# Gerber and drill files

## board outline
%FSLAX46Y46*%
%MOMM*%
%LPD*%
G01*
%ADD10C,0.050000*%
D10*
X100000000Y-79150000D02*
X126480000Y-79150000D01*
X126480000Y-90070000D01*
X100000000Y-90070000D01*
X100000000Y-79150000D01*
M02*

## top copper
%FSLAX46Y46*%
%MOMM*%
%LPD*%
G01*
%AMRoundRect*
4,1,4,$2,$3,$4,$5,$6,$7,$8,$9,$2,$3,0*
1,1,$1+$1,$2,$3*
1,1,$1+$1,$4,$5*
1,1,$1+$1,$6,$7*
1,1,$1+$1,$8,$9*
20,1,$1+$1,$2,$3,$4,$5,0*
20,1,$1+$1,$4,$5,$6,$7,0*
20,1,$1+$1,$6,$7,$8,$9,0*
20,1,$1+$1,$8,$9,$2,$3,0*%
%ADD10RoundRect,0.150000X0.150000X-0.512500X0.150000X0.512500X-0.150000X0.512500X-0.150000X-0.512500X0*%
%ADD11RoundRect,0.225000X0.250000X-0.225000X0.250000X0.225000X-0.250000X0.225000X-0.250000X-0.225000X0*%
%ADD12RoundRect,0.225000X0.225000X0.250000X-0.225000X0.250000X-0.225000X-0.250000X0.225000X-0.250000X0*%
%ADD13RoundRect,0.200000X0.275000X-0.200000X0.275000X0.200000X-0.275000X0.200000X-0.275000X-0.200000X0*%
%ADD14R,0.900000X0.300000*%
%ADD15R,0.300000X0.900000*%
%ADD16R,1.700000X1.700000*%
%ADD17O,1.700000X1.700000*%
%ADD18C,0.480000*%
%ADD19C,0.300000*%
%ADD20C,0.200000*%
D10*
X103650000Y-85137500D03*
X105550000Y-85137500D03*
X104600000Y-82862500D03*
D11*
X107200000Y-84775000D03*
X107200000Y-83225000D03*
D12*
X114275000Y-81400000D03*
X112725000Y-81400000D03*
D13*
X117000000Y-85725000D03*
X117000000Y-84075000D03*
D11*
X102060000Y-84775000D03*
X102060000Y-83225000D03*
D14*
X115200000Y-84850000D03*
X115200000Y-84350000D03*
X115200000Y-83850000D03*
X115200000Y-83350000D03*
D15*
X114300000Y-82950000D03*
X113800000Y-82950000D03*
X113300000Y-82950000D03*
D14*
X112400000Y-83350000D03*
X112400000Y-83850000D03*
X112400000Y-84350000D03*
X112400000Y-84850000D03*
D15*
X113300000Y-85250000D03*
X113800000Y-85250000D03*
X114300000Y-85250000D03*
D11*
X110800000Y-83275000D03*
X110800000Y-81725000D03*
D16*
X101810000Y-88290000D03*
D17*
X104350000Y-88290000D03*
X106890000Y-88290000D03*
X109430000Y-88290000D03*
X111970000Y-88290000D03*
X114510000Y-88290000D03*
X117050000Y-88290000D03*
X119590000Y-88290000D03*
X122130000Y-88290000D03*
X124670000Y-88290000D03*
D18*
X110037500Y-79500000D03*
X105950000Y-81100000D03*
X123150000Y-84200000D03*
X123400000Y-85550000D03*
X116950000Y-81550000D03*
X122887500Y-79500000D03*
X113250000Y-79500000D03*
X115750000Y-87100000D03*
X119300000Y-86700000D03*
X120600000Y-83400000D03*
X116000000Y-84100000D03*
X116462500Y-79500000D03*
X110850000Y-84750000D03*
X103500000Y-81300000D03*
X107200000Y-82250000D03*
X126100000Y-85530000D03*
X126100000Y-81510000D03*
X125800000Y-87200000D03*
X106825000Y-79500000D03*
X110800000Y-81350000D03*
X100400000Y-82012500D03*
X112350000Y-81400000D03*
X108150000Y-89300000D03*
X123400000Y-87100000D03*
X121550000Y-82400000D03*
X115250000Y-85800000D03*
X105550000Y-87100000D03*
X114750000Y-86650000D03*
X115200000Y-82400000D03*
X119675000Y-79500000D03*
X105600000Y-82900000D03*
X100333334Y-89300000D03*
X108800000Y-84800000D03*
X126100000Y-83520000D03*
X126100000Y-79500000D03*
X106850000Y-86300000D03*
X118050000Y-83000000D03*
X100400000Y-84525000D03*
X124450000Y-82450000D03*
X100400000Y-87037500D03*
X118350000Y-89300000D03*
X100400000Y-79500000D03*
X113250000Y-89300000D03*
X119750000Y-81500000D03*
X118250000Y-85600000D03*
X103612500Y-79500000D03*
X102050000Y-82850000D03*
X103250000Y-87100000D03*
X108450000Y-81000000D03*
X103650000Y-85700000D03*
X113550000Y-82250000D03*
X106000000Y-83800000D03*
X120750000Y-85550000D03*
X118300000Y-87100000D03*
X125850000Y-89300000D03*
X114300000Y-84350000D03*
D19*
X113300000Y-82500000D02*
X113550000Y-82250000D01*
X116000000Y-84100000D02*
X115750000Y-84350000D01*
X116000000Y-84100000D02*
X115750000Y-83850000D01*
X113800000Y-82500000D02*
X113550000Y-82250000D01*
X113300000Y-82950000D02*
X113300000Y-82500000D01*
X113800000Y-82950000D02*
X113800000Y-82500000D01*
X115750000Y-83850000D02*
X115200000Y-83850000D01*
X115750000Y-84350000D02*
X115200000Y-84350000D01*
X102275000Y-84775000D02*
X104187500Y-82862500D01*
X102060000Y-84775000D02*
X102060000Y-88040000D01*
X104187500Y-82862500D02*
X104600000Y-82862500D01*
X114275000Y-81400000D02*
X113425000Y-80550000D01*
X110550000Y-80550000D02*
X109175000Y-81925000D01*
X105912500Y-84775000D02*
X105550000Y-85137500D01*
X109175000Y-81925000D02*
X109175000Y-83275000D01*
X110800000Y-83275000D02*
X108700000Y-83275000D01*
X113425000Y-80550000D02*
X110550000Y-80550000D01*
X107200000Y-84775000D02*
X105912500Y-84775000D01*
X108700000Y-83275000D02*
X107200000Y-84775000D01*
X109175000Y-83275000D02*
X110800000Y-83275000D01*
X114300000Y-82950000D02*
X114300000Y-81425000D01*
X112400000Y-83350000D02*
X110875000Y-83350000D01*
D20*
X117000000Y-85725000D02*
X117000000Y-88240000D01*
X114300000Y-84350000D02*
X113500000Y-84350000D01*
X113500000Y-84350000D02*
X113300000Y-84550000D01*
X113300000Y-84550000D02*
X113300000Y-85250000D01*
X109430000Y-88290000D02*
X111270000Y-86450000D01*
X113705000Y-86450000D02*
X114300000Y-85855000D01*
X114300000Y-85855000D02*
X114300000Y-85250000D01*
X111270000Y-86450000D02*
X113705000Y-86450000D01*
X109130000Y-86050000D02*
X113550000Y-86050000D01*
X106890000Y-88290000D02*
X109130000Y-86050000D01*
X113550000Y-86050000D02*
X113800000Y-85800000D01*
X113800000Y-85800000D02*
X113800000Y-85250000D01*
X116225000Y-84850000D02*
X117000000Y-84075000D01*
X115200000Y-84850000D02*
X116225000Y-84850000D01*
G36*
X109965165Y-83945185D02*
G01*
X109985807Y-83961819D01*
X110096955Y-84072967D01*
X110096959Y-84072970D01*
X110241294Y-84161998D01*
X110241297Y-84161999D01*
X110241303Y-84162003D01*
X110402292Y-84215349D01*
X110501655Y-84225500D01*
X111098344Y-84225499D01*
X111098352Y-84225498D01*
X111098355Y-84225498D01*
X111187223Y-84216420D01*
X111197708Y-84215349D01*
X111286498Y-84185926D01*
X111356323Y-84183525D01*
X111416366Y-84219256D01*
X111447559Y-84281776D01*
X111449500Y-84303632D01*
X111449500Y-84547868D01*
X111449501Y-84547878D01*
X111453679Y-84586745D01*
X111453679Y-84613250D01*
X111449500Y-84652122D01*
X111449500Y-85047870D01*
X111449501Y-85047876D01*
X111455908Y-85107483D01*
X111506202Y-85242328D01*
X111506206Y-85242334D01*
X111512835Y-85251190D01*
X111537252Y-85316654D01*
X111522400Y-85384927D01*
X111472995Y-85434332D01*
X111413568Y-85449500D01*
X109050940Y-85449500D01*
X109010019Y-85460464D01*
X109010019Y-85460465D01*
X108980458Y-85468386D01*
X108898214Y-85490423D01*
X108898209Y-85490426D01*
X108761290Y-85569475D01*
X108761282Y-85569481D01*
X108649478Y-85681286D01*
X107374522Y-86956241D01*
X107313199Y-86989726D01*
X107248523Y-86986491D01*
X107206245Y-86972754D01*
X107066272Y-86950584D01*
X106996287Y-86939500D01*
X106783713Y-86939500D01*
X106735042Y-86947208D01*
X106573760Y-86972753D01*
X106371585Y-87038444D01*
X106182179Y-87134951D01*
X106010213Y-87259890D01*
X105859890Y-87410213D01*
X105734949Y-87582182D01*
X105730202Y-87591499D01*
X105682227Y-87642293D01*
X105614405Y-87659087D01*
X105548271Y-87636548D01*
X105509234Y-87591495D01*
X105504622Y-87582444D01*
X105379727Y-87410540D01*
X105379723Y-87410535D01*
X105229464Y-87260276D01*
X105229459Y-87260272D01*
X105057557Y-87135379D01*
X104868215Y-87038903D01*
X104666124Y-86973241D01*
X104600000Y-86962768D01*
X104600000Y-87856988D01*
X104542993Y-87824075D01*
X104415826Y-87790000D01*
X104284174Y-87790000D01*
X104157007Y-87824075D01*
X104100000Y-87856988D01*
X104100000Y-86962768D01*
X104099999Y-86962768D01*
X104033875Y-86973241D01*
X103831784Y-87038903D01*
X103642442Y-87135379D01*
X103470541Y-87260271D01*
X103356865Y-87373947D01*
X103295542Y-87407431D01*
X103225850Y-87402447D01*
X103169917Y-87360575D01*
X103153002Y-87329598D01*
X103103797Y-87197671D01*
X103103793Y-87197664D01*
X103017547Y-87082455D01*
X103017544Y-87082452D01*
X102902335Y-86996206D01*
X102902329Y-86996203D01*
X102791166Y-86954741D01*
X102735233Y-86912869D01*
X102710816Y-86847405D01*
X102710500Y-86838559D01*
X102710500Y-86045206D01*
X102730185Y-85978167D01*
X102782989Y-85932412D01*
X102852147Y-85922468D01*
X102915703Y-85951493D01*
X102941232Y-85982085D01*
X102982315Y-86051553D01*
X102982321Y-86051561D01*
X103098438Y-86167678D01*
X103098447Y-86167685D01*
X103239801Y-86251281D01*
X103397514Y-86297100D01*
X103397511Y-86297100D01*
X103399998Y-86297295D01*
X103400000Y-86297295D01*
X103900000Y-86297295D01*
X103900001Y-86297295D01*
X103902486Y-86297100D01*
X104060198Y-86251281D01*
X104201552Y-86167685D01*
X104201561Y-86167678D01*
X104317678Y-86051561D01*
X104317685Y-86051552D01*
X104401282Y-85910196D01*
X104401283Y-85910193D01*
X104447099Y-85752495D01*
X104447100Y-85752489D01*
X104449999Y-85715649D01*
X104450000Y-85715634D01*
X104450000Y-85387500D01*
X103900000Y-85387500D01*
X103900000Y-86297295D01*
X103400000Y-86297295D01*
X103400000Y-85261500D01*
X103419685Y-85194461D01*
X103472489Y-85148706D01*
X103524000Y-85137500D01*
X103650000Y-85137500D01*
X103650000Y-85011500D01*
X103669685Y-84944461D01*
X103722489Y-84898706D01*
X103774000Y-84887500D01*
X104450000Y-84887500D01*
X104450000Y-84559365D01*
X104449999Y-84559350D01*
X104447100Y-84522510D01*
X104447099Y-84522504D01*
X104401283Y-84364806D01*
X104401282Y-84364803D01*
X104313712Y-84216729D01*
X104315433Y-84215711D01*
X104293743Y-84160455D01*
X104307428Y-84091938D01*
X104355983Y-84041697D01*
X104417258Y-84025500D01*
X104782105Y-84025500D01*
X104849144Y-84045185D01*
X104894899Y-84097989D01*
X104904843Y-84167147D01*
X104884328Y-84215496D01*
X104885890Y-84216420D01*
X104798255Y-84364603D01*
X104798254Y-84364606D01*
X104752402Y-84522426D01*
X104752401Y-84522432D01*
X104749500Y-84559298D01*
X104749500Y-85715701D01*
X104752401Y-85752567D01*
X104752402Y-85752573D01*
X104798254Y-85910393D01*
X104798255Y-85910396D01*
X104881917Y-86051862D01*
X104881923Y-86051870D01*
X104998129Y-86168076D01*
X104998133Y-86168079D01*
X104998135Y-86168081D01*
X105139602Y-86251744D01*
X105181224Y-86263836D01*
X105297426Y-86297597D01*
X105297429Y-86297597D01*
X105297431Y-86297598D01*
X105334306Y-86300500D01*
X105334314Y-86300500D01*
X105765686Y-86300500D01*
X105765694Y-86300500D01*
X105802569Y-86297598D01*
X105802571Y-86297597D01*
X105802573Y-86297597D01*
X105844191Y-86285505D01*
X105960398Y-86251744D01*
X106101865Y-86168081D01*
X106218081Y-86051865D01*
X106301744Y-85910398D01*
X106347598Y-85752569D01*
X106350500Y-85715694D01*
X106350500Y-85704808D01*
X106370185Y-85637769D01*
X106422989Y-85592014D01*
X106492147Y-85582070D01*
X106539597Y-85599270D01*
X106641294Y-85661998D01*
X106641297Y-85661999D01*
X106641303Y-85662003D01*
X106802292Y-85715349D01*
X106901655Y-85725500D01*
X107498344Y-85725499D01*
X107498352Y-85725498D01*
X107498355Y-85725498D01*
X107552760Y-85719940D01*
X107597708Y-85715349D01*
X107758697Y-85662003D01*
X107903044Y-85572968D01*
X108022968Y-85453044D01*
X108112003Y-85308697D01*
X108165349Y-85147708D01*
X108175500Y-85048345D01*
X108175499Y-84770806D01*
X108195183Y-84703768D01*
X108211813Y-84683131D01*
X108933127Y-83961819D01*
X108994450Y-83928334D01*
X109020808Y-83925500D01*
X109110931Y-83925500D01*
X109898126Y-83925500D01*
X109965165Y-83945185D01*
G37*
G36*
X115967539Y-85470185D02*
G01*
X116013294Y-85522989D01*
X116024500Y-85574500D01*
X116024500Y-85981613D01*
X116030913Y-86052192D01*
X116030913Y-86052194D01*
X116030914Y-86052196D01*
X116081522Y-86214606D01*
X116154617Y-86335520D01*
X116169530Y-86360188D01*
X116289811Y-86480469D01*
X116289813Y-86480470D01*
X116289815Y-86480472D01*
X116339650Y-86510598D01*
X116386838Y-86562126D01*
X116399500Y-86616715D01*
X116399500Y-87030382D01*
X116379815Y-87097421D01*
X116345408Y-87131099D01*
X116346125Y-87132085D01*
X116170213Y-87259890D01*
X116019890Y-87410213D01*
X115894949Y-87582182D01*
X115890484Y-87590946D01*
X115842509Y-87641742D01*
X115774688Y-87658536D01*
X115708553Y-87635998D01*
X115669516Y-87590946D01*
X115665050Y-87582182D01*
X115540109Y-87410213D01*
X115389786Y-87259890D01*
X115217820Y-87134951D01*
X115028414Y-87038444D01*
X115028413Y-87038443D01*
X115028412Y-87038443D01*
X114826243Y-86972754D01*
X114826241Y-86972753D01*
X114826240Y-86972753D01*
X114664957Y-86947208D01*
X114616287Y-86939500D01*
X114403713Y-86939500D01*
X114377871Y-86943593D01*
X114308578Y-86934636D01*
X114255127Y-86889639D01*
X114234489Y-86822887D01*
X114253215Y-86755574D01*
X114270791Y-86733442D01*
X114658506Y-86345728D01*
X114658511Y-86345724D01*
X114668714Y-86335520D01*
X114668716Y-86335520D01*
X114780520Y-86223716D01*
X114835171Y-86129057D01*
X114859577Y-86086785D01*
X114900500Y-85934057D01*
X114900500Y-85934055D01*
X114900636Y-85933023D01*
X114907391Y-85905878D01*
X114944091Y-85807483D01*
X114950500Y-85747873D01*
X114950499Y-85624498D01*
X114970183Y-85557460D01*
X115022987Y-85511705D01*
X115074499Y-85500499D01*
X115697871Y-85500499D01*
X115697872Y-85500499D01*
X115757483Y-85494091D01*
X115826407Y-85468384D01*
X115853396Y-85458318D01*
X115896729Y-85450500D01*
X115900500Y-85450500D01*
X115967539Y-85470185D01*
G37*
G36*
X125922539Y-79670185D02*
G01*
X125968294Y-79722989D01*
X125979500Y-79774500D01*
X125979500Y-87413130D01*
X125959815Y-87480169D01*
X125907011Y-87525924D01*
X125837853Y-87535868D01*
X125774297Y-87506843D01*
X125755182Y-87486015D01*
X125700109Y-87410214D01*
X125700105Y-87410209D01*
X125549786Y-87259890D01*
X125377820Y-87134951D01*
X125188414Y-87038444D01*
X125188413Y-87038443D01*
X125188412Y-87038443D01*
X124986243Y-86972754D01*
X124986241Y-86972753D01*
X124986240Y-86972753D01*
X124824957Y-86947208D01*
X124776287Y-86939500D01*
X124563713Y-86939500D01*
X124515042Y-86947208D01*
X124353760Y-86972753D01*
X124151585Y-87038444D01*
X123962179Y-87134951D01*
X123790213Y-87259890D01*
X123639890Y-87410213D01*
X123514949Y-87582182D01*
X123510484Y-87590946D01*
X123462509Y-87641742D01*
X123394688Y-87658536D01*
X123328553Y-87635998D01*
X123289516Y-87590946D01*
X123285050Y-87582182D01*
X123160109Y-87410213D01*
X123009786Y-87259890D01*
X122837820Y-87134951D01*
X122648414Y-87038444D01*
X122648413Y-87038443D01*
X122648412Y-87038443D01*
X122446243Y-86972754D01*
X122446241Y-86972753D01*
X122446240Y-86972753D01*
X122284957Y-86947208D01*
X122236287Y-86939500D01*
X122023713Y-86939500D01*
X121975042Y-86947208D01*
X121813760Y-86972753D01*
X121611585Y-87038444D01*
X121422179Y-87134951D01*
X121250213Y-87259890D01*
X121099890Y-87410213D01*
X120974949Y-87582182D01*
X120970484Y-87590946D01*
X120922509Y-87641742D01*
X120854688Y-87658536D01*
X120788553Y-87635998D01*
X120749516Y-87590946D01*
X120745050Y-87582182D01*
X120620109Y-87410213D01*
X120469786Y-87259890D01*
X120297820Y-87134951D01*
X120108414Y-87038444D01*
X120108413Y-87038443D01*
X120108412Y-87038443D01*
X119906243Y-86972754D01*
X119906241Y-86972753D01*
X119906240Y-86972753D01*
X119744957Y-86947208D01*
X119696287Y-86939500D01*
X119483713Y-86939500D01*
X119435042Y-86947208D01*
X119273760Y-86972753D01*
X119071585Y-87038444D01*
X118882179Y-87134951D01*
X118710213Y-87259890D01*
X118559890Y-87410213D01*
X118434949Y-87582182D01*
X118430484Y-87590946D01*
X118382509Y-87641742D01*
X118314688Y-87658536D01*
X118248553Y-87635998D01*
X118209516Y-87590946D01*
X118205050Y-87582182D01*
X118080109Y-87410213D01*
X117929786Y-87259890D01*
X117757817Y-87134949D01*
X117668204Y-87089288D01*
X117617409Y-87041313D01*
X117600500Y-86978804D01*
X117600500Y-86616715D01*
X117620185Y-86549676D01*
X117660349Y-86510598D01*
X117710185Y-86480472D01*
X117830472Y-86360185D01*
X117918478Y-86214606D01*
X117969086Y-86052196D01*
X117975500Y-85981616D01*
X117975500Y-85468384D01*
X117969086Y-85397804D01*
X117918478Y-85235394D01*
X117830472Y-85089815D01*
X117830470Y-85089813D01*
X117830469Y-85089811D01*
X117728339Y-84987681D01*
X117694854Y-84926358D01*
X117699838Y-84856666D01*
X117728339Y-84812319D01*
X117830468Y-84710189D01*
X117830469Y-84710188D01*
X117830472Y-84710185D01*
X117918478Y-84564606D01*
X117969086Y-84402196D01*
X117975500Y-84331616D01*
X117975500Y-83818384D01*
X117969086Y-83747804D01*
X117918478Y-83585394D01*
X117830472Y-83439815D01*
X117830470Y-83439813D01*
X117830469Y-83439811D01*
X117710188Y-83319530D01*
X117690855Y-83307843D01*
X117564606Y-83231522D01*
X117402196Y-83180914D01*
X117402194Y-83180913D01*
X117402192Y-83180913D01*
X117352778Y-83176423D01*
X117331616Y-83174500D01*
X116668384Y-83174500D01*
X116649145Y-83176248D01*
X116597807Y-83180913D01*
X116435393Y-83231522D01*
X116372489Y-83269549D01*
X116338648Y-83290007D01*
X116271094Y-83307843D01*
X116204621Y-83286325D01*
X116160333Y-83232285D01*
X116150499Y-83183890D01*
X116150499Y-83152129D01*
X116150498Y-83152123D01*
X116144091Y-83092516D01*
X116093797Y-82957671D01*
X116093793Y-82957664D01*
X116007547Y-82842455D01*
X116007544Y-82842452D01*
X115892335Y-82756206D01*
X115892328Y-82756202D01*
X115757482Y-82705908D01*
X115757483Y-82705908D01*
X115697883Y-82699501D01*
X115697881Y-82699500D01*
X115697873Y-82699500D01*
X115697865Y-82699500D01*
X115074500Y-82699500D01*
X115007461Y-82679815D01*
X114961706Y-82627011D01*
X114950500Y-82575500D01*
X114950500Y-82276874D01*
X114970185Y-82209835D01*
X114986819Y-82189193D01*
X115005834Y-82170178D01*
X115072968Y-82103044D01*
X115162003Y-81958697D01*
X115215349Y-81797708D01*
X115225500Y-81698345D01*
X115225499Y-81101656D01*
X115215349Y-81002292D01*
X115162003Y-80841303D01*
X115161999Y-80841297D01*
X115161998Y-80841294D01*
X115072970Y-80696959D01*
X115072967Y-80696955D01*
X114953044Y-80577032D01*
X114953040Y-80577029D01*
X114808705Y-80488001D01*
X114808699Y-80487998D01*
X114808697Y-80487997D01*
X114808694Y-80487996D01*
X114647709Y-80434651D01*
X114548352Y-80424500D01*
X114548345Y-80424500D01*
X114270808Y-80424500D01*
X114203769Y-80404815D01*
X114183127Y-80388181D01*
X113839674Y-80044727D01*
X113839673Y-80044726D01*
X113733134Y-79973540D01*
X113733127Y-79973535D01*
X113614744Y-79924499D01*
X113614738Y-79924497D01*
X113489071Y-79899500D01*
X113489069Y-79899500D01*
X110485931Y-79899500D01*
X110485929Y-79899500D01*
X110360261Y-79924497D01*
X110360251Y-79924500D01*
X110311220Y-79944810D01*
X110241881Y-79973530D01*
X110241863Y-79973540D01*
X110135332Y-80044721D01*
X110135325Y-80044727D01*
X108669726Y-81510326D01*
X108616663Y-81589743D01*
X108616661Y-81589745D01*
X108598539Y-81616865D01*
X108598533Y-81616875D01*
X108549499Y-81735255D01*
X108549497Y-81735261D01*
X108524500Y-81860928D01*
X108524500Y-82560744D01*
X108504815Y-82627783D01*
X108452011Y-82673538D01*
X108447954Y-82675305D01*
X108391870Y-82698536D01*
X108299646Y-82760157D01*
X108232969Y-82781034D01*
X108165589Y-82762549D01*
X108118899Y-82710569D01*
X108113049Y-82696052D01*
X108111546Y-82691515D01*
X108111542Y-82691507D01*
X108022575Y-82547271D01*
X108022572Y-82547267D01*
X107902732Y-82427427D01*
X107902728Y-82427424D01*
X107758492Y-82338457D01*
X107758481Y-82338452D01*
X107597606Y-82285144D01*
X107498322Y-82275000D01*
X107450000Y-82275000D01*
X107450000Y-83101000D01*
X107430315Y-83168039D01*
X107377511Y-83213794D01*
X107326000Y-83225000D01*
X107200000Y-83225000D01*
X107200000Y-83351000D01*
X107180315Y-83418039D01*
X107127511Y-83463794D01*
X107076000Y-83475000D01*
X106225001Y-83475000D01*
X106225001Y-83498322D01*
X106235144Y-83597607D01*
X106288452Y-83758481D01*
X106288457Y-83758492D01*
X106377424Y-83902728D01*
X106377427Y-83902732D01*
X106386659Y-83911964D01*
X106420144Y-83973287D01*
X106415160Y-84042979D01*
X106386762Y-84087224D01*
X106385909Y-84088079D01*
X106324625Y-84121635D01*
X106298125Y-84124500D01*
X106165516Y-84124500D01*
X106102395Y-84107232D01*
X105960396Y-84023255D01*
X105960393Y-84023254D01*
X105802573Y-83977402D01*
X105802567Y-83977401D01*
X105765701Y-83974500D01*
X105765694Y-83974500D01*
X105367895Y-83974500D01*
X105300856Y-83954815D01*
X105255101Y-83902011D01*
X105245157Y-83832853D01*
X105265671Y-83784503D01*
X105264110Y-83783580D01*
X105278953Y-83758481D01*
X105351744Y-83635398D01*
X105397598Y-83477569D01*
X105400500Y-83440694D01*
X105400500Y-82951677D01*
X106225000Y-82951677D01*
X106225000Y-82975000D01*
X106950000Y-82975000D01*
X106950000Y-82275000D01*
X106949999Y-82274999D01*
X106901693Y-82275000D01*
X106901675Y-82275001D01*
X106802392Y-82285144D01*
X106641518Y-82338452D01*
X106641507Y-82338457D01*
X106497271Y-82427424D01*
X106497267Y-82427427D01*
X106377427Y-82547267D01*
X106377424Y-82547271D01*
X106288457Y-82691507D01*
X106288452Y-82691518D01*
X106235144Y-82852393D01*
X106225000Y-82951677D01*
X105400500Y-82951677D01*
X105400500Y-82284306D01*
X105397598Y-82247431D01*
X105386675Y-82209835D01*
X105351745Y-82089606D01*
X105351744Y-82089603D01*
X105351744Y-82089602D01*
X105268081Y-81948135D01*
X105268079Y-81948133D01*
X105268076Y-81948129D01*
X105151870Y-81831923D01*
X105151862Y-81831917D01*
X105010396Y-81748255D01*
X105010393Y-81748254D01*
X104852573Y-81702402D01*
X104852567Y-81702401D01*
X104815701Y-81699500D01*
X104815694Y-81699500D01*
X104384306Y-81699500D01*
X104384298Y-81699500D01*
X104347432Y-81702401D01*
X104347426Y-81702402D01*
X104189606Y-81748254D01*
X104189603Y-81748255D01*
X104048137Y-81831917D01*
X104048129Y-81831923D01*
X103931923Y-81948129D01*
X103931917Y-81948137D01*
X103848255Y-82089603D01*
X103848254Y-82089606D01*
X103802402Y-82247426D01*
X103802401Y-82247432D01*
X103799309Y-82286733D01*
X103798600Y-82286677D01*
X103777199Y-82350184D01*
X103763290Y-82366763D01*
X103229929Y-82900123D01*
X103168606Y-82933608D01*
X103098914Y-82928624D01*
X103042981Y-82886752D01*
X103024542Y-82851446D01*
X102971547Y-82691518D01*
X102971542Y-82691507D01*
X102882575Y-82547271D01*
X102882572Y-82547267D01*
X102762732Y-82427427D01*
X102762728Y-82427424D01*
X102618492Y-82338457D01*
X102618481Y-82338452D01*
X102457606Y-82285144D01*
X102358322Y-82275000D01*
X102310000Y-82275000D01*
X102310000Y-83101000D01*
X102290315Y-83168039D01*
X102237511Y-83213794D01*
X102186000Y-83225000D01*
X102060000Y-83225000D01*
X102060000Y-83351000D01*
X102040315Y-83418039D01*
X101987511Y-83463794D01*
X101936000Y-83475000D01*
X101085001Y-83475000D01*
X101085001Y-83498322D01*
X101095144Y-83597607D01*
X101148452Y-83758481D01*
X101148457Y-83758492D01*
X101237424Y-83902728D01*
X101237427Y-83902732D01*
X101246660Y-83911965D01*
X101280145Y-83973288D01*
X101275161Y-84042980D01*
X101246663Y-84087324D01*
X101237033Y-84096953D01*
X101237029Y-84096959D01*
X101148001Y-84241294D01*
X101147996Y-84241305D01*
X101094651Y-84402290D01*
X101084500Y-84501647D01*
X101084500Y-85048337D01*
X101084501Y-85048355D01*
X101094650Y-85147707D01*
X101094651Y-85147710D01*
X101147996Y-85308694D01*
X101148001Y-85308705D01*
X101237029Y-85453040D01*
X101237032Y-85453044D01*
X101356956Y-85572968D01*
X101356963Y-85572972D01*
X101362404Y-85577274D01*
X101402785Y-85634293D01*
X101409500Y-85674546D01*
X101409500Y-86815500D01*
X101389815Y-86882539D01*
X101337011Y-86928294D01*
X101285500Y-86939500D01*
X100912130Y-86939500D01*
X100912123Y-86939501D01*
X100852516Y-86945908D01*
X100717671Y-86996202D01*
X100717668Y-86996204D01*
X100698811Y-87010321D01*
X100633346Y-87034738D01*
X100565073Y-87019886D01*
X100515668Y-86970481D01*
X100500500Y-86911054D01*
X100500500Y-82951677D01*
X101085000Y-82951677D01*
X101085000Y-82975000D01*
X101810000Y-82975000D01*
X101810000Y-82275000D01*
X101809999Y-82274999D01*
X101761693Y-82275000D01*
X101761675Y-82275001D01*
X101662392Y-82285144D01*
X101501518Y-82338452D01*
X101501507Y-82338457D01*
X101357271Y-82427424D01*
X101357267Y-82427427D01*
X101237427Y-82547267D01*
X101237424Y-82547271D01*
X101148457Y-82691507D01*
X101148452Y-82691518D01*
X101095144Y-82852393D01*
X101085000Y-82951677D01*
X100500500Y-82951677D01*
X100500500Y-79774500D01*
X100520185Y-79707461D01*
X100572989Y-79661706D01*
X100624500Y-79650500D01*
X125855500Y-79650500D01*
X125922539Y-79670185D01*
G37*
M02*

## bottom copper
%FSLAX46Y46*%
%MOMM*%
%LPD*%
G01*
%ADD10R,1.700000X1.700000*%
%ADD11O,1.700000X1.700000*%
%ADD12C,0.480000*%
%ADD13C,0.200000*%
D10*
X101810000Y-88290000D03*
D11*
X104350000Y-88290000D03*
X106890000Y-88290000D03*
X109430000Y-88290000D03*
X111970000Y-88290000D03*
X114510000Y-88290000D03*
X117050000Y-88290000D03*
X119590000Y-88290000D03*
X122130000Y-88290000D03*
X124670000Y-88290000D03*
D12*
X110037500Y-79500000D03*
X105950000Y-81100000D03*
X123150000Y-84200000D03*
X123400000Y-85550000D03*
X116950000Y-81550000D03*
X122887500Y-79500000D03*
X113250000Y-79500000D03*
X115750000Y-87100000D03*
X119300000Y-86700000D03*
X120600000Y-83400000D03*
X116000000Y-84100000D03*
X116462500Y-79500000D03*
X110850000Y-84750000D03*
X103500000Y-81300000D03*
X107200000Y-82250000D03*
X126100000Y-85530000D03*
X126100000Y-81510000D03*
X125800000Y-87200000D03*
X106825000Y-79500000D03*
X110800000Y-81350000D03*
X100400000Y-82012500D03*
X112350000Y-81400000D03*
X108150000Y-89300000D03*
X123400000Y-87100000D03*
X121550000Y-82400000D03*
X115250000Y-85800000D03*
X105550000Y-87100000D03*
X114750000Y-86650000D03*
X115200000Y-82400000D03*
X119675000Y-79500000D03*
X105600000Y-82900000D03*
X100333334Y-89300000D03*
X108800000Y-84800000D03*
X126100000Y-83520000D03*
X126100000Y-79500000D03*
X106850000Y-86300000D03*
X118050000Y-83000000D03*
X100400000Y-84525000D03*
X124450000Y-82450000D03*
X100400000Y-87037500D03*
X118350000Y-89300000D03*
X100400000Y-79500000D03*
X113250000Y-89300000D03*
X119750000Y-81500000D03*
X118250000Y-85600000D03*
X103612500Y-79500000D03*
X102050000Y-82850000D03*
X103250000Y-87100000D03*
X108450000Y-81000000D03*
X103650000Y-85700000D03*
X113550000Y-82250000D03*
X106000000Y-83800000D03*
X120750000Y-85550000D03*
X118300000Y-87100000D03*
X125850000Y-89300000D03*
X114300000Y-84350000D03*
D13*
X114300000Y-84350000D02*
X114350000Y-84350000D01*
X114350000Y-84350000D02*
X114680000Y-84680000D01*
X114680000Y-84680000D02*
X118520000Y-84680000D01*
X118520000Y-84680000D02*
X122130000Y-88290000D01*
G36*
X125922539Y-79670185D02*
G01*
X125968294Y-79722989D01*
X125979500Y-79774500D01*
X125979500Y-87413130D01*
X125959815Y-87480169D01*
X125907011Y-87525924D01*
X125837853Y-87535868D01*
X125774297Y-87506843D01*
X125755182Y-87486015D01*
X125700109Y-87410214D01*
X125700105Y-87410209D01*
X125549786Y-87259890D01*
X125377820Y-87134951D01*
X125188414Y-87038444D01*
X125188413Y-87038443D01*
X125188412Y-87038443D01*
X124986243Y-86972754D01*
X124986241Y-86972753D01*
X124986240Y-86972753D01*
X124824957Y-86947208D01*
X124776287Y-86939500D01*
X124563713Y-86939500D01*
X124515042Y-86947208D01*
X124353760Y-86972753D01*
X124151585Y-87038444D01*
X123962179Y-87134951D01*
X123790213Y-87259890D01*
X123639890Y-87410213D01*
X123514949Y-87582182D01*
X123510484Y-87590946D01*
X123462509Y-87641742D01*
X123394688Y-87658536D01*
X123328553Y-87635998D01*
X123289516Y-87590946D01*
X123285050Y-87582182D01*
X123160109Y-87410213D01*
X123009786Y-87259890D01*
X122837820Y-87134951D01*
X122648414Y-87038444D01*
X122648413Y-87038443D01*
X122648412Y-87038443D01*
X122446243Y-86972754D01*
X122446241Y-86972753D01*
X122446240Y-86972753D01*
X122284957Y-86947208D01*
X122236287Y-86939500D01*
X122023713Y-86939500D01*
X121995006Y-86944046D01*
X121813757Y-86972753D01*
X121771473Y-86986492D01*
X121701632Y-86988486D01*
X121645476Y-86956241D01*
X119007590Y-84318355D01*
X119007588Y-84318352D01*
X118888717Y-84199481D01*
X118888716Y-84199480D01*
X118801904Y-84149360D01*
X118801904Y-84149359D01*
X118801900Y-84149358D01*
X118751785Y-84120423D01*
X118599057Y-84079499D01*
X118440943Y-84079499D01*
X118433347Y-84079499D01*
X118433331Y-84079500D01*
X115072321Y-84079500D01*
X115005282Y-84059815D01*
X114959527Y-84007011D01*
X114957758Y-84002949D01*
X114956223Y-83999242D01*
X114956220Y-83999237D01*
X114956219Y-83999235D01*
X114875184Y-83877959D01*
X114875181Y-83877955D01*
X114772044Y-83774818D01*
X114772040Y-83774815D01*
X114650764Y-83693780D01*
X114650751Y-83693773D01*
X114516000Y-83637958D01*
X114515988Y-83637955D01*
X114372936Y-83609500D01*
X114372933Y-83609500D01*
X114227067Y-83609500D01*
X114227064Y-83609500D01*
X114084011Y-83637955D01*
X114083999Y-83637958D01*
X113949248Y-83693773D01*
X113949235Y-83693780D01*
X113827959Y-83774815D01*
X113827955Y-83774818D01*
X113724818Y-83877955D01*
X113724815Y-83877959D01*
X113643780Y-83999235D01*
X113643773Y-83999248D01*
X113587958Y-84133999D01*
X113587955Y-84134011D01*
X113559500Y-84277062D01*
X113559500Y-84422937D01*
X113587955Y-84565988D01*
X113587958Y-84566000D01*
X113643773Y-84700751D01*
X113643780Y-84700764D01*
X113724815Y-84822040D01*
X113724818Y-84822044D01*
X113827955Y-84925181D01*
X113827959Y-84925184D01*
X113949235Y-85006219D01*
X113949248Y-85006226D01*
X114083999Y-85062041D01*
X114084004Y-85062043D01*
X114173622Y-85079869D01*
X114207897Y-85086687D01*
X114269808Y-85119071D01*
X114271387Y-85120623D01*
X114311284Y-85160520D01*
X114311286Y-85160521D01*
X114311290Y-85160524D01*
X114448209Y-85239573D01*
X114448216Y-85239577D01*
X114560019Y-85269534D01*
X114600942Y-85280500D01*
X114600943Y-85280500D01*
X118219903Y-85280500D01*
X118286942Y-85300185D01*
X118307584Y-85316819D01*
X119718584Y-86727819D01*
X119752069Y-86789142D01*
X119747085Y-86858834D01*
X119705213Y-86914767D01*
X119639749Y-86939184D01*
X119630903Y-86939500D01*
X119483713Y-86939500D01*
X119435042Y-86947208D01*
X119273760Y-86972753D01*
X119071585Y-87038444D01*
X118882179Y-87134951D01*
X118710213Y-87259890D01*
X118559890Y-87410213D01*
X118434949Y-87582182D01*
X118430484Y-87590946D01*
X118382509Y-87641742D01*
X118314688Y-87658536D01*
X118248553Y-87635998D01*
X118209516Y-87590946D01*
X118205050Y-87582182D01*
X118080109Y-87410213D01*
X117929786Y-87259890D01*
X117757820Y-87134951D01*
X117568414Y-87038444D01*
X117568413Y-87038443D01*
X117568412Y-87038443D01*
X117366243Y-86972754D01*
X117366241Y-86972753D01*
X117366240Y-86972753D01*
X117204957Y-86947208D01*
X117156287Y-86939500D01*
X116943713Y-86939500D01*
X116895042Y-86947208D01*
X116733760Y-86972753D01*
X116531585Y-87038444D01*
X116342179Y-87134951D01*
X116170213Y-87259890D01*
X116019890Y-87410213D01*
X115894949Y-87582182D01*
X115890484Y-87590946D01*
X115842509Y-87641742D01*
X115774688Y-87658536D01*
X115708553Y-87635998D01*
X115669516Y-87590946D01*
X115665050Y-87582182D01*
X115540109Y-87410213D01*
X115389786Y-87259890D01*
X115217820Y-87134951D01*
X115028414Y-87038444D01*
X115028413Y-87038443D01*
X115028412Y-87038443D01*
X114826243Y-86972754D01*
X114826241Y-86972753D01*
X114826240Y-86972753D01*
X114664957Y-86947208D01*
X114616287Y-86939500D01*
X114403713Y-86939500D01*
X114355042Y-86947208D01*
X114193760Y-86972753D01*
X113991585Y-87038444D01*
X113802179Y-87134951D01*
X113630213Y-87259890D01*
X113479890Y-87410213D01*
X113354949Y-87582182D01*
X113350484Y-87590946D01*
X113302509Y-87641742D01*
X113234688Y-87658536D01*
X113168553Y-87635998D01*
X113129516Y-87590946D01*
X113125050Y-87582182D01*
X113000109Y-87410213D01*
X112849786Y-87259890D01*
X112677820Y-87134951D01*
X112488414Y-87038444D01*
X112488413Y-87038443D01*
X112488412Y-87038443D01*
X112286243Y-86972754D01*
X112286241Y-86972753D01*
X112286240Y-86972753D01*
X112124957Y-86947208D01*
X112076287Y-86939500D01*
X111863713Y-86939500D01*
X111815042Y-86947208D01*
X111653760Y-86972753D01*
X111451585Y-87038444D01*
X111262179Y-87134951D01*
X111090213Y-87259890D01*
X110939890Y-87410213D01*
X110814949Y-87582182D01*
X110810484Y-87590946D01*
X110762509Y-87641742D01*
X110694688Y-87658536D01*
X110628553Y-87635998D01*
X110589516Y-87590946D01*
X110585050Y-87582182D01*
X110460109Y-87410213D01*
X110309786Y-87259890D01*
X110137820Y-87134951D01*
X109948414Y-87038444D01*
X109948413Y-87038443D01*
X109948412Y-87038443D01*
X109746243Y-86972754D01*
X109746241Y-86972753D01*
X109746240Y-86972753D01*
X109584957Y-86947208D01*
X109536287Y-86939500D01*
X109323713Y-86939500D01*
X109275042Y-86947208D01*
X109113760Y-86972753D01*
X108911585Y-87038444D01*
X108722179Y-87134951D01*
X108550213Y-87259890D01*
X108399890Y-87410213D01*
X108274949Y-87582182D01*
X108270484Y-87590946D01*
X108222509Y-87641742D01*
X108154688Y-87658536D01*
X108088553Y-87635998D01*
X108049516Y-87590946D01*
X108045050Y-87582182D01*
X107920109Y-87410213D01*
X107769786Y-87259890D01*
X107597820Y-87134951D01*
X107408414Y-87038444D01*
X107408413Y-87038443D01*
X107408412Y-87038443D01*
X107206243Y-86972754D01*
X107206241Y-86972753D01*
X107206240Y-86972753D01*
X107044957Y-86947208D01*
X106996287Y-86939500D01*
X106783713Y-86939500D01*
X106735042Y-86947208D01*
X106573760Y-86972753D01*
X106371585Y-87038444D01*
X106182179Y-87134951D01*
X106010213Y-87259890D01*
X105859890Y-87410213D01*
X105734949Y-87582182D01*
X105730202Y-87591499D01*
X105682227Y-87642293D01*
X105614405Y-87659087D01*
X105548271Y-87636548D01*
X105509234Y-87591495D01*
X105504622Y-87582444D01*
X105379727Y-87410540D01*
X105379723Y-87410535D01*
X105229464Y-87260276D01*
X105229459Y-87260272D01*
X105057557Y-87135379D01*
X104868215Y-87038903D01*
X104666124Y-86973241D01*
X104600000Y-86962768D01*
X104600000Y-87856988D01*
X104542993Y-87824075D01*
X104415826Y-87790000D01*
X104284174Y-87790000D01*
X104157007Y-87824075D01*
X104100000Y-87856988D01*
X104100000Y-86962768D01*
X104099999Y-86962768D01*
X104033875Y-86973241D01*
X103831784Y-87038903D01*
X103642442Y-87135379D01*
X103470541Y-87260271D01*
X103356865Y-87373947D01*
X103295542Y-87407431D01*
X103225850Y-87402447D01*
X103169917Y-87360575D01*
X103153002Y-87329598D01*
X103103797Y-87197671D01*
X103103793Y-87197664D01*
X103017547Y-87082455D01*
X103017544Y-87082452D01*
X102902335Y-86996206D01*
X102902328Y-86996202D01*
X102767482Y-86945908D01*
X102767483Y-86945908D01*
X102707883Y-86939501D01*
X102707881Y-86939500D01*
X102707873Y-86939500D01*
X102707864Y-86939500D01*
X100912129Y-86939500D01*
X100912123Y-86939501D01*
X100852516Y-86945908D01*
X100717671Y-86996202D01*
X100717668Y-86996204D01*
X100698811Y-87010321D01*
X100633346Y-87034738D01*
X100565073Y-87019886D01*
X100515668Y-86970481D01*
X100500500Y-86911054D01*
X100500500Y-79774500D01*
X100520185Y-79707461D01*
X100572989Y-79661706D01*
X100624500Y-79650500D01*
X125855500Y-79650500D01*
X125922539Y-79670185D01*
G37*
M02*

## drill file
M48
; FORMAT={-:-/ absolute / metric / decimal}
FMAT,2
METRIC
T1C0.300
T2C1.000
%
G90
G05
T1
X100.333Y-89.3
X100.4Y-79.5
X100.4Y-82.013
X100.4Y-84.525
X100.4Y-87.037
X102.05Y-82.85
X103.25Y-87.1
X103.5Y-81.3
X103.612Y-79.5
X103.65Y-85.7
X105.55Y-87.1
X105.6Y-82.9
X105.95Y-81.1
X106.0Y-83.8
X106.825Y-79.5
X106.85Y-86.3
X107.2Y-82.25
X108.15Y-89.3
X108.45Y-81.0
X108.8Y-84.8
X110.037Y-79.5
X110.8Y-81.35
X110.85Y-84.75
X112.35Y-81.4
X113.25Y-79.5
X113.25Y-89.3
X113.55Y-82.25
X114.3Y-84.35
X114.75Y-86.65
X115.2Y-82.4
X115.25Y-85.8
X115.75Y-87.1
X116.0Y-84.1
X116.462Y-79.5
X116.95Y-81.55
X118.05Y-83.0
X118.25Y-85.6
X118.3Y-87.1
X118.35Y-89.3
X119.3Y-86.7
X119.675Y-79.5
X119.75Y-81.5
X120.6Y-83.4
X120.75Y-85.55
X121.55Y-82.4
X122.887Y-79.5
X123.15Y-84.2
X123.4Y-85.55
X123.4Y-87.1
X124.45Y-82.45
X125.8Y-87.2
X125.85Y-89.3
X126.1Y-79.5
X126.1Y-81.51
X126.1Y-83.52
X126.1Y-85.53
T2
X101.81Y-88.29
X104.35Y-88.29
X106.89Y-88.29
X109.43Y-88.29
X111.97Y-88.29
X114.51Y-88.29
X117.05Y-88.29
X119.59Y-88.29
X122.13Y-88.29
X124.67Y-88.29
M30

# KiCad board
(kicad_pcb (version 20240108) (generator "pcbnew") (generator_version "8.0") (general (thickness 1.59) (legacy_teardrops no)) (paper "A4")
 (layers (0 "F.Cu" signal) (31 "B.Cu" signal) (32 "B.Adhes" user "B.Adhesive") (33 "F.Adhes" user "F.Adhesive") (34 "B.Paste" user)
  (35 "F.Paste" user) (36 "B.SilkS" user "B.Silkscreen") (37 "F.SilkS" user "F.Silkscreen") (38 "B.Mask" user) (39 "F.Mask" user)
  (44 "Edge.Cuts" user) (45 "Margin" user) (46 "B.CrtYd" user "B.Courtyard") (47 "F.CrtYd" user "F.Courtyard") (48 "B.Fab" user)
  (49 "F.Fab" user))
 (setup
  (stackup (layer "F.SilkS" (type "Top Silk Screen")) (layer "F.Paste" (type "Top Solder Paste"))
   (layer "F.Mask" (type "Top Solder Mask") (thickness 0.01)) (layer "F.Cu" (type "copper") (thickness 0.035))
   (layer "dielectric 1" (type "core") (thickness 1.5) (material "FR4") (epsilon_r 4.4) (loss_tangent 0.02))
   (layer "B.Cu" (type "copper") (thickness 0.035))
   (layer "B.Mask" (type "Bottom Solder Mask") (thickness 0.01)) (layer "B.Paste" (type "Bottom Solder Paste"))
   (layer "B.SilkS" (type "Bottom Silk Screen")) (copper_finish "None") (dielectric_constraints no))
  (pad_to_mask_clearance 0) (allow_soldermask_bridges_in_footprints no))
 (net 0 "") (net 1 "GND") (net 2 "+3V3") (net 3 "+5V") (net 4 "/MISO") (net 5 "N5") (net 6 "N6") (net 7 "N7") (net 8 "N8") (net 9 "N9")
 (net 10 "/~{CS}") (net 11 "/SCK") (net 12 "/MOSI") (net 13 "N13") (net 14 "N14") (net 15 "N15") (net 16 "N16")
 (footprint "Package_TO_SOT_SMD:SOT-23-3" (layer "F.Cu") (at 104.6 84 90)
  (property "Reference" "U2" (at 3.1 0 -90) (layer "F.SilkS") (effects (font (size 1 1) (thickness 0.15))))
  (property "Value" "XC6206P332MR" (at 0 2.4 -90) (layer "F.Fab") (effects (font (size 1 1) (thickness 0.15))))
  (pad "1" smd roundrect (at -1.1375 -0.95 90) (size 1.325 0.6) (layers "F.Cu" "F.Paste" "F.Mask") (roundrect_rratio 0.25) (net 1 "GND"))
  (pad "2" smd roundrect (at -1.1375 0.95 90) (size 1.325 0.6) (layers "F.Cu" "F.Paste" "F.Mask") (roundrect_rratio 0.25) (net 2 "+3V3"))
  (pad "3" smd roundrect (at 1.1375 0 90) (size 1.325 0.6) (layers "F.Cu" "F.Paste" "F.Mask") (roundrect_rratio 0.25) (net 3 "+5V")))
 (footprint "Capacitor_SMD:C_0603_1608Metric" (layer "F.Cu") (at 107.2 84 90)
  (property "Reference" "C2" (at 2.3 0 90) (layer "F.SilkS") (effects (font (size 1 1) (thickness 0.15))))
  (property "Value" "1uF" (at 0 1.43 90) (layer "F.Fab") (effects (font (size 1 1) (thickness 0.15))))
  (pad "1" smd roundrect (at -0.775 0 90) (size 0.9 0.95) (layers "F.Cu" "F.Paste" "F.Mask") (roundrect_rratio 0.25) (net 2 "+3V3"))
  (pad "2" smd roundrect (at 0.775 0 90) (size 0.9 0.95) (layers "F.Cu" "F.Paste" "F.Mask") (roundrect_rratio 0.25) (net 1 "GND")))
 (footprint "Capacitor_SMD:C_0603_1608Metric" (layer "F.Cu") (at 113.5 81.4 180)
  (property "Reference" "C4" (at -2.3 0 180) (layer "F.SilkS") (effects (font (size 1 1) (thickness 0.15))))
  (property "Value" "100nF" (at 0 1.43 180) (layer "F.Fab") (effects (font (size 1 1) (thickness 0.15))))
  (pad "1" smd roundrect (at -0.775 0 180) (size 0.9 0.95) (layers "F.Cu" "F.Paste" "F.Mask") (roundrect_rratio 0.25) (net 2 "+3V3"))
  (pad "2" smd roundrect (at 0.775 0 180) (size 0.9 0.95) (layers "F.Cu" "F.Paste" "F.Mask") (roundrect_rratio 0.25) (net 1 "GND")))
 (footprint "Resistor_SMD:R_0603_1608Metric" (layer "F.Cu") (at 117 84.9 90)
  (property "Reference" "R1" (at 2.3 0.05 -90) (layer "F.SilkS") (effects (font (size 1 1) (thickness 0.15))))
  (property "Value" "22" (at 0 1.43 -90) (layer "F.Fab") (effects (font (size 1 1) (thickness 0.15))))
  (pad "1" smd roundrect (at -0.825 0 90) (size 0.8 0.95) (layers "F.Cu" "F.Paste" "F.Mask") (roundrect_rratio 0.25) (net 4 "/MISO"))
  (pad "2" smd roundrect (at 0.825 0 90) (size 0.8 0.95) (layers "F.Cu" "F.Paste" "F.Mask") (roundrect_rratio 0.25) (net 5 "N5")))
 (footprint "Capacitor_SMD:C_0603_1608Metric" (layer "F.Cu") (at 102.06 84 90)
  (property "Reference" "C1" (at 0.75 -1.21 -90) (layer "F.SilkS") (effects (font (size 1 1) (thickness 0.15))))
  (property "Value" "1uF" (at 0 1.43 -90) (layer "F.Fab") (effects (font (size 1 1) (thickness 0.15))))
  (pad "1" smd roundrect (at -0.775 0 90) (size 0.9 0.95) (layers "F.Cu" "F.Paste" "F.Mask") (roundrect_rratio 0.25) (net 3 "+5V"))
  (pad "2" smd roundrect (at 0.775 0 90) (size 0.9 0.95) (layers "F.Cu" "F.Paste" "F.Mask") (roundrect_rratio 0.25) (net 1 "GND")))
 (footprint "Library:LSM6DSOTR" (layer "F.Cu") (at 113.8 84.1 180)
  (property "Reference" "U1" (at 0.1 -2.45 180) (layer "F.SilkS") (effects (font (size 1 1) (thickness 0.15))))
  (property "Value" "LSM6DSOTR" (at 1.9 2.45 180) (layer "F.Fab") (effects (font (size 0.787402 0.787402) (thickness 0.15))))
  (pad "1" smd rect (at -1.4 -0.75 180) (size 0.9 0.3) (layers "F.Cu") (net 5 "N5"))
  (pad "2" smd rect (at -1.4 -0.25 180) (size 0.9 0.3) (layers "F.Cu") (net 1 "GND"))
  (pad "3" smd rect (at -1.4 0.25 180) (size 0.9 0.3) (layers "F.Cu") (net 1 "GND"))
  (pad "4" smd rect (at -1.4 0.75 180) (size 0.9 0.3) (layers "F.Cu") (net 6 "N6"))
  (pad "5" smd rect (at -0.5 1.15 180) (size 0.3 0.9) (layers "F.Cu") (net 2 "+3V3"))
  (pad "6" smd rect (at 0 1.15 180) (size 0.3 0.9) (layers "F.Cu") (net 1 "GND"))
  (pad "7" smd rect (at 0.5 1.15 180) (size 0.3 0.9) (layers "F.Cu") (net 1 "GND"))
  (pad "8" smd rect (at 1.4 0.75 180) (size 0.9 0.3) (layers "F.Cu") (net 2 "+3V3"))
  (pad "9" smd rect (at 1.4 0.25 180) (size 0.9 0.3) (layers "F.Cu") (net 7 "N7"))
  (pad "10" smd rect (at 1.4 -0.25 180) (size 0.9 0.3) (layers "F.Cu") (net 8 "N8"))
  (pad "11" smd rect (at 1.4 -0.75 180) (size 0.9 0.3) (layers "F.Cu") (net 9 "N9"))
  (pad "12" smd rect (at 0.5 -1.15 180) (size 0.3 0.9) (layers "F.Cu") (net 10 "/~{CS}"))
  (pad "13" smd rect (at 0 -1.15 180) (size 0.3 0.9) (layers "F.Cu") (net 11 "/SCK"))
  (pad "14" smd rect (at -0.5 -1.15 180) (size 0.3 0.9) (layers "F.Cu") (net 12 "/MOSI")))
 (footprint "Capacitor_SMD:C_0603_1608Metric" (layer "F.Cu") (at 110.8 82.5 90)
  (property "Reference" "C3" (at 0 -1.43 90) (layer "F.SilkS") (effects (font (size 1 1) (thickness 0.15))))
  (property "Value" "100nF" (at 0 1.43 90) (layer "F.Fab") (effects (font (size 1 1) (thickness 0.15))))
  (pad "1" smd roundrect (at -0.775 0 90) (size 0.9 0.95) (layers "F.Cu" "F.Paste" "F.Mask") (roundrect_rratio 0.25) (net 2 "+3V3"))
  (pad "2" smd roundrect (at 0.775 0 90) (size 0.9 0.95) (layers "F.Cu" "F.Paste" "F.Mask") (roundrect_rratio 0.25) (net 1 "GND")))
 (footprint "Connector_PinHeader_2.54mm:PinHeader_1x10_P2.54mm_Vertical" (layer "B.Cu") (at 101.81 88.29 -90)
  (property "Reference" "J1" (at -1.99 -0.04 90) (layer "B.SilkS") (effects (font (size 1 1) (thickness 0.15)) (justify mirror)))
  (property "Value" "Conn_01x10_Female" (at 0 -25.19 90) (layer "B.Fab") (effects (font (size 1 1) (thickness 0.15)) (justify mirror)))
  (pad "1" thru_hole rect (at 0 0 270) (size 1.7 1.7) (drill 1) (layers "*.Cu" "*.Mask") (remove_unused_layers no) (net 3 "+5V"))
  (pad "2" thru_hole oval (at 0 -2.54 270) (size 1.7 1.7) (drill 1) (layers "*.Cu" "*.Mask") (remove_unused_layers no) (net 1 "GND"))
  (pad "3" thru_hole oval (at 0 -5.08 270) (size 1.7 1.7) (drill 1) (layers "*.Cu" "*.Mask") (remove_unused_layers no) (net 11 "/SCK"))
  (pad "4" thru_hole oval (at 0 -7.62 270) (size 1.7 1.7) (drill 1) (layers "*.Cu" "*.Mask") (remove_unused_layers no) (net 12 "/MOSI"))
  (pad "5" thru_hole oval (at 0 -10.16 270) (size 1.7 1.7) (drill 1) (layers "*.Cu" "*.Mask") (remove_unused_layers no) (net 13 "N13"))
  (pad "6" thru_hole oval (at 0 -12.7 270) (size 1.7 1.7) (drill 1) (layers "*.Cu" "*.Mask") (remove_unused_layers no) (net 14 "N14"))
  (pad "7" thru_hole oval (at 0 -15.24 270) (size 1.7 1.7) (drill 1) (layers "*.Cu" "*.Mask") (remove_unused_layers no) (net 4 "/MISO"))
  (pad "8" thru_hole oval (at 0 -17.78 270) (size 1.7 1.7) (drill 1) (layers "*.Cu" "*.Mask") (remove_unused_layers no) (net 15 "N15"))
  (pad "9" thru_hole oval (at 0 -20.32 270) (size 1.7 1.7) (drill 1) (layers "*.Cu" "*.Mask") (remove_unused_layers no) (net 10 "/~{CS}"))
  (pad "10" thru_hole oval (at 0 -22.86 270) (size 1.7 1.7) (drill 1) (layers "*.Cu" "*.Mask") (remove_unused_layers no) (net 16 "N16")))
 (gr_rect (start 100 79.15) (end 126.48 90.07) (stroke (width 0.05) (type default)) (fill none) (layer "Edge.Cuts"))
 (segment (start 113.3 82.5) (end 113.55 82.25) (width 0.3) (layer "F.Cu") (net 1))
 (segment (start 116 84.1) (end 115.75 84.35) (width 0.3) (layer "F.Cu") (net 1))
 (segment (start 116 84.1) (end 115.75 83.85) (width 0.3) (layer "F.Cu") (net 1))
 (segment (start 113.8 82.5) (end 113.55 82.25) (width 0.3) (layer "F.Cu") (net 1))
 (segment (start 113.3 82.95) (end 113.3 82.5) (width 0.3) (layer "F.Cu") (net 1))
 (segment (start 113.8 82.95) (end 113.8 82.5) (width 0.3) (layer "F.Cu") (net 1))
 (segment (start 115.75 83.85) (end 115.2 83.85) (width 0.3) (layer "F.Cu") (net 1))
 (segment (start 115.75 84.35) (end 115.2 84.35) (width 0.3) (layer "F.Cu") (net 1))
 (via (at 110.0375 79.5) (size 0.48) (drill 0.3) (layers "F.Cu" "B.Cu") (free yes) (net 1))
 (via (at 105.95 81.1) (size 0.48) (drill 0.3) (layers "F.Cu" "B.Cu") (free yes) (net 1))
 (via (at 123.15 84.2) (size 0.48) (drill 0.3) (layers "F.Cu" "B.Cu") (free yes) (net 1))
 (via (at 123.4 85.55) (size 0.48) (drill 0.3) (layers "F.Cu" "B.Cu") (free yes) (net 1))
 (via (at 116.95 81.55) (size 0.48) (drill 0.3) (layers "F.Cu" "B.Cu") (free yes) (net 1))
 (via (at 122.8875 79.5) (size 0.48) (drill 0.3) (layers "F.Cu" "B.Cu") (free yes) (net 1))
 (via (at 113.25 79.5) (size 0.48) (drill 0.3) (layers "F.Cu" "B.Cu") (free yes) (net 1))
 (via (at 115.75 87.1) (size 0.48) (drill 0.3) (layers "F.Cu" "B.Cu") (free yes) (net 1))
 (via (at 119.3 86.7) (size 0.48) (drill 0.3) (layers "F.Cu" "B.Cu") (free yes) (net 1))
 (via (at 120.6 83.4) (size 0.48) (drill 0.3) (layers "F.Cu" "B.Cu") (free yes) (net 1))
 (via (at 116 84.1) (size 0.48) (drill 0.3) (layers "F.Cu" "B.Cu") (free yes) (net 1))
 (via (at 116.4625 79.5) (size 0.48) (drill 0.3) (layers "F.Cu" "B.Cu") (free yes) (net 1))
 (via (at 110.85 84.75) (size 0.48) (drill 0.3) (layers "F.Cu" "B.Cu") (free yes) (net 1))
 (via (at 103.5 81.3) (size 0.48) (drill 0.3) (layers "F.Cu" "B.Cu") (free yes) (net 1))
 (via (at 107.2 82.25) (size 0.48) (drill 0.3) (layers "F.Cu" "B.Cu") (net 1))
 (via (at 126.1 85.53) (size 0.48) (drill 0.3) (layers "F.Cu" "B.Cu") (free yes) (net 1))
 (via (at 126.1 81.51) (size 0.48) (drill 0.3) (layers "F.Cu" "B.Cu") (free yes) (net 1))
 (via (at 125.8 87.2) (size 0.48) (drill 0.3) (layers "F.Cu" "B.Cu") (free yes) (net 1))
 (via (at 106.825 79.5) (size 0.48) (drill 0.3) (layers "F.Cu" "B.Cu") (free yes) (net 1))
 (via (at 110.8 81.35) (size 0.48) (drill 0.3) (layers "F.Cu" "B.Cu") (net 1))
 (via (at 100.4 82.0125) (size 0.48) (drill 0.3) (layers "F.Cu" "B.Cu") (free yes) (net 1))
 (via (at 112.35 81.4) (size 0.48) (drill 0.3) (layers "F.Cu" "B.Cu") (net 1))
 (via (at 108.15 89.3) (size 0.48) (drill 0.3) (layers "F.Cu" "B.Cu") (free yes) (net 1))
 (via (at 123.4 87.1) (size 0.48) (drill 0.3) (layers "F.Cu" "B.Cu") (free yes) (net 1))
 (via (at 121.55 82.4) (size 0.48) (drill 0.3) (layers "F.Cu" "B.Cu") (free yes) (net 1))
 (via (at 115.25 85.8) (size 0.48) (drill 0.3) (layers "F.Cu" "B.Cu") (free yes) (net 1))
 (via (at 105.55 87.1) (size 0.48) (drill 0.3) (layers "F.Cu" "B.Cu") (free yes) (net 1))
 (via (at 114.75 86.65) (size 0.48) (drill 0.3) (layers "F.Cu" "B.Cu") (free yes) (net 1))
 (via (at 115.2 82.4) (size 0.48) (drill 0.3) (layers "F.Cu" "B.Cu") (free yes) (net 1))
 (via (at 119.675 79.5) (size 0.48) (drill 0.3) (layers "F.Cu" "B.Cu") (free yes) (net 1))
 (via (at 105.6 82.9) (size 0.48) (drill 0.3) (layers "F.Cu" "B.Cu") (free yes) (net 1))
 (via (at 100.333334 89.3) (size 0.48) (drill 0.3) (layers "F.Cu" "B.Cu") (free yes) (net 1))
 (via (at 108.8 84.8) (size 0.48) (drill 0.3) (layers "F.Cu" "B.Cu") (free yes) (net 1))
 (via (at 126.1 83.52) (size 0.48) (drill 0.3) (layers "F.Cu" "B.Cu") (free yes) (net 1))
 (via (at 126.1 79.5) (size 0.48) (drill 0.3) (layers "F.Cu" "B.Cu") (free yes) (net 1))
 (via (at 106.85 86.3) (size 0.48) (drill 0.3) (layers "F.Cu" "B.Cu") (free yes) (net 1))
 (via (at 118.05 83) (size 0.48) (drill 0.3) (layers "F.Cu" "B.Cu") (free yes) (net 1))
 (via (at 100.4 84.525) (size 0.48) (drill 0.3) (layers "F.Cu" "B.Cu") (free yes) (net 1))
 (via (at 124.45 82.45) (size 0.48) (drill 0.3) (layers "F.Cu" "B.Cu") (free yes) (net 1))
 (via (at 100.4 87.0375) (size 0.48) (drill 0.3) (layers "F.Cu" "B.Cu") (free yes) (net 1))
 (via (at 118.35 89.3) (size 0.48) (drill 0.3) (layers "F.Cu" "B.Cu") (free yes) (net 1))
 (via (at 100.4 79.5) (size 0.48) (drill 0.3) (layers "F.Cu" "B.Cu") (free yes) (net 1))
 (via (at 113.25 89.3) (size 0.48) (drill 0.3) (layers "F.Cu" "B.Cu") (free yes) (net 1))
 (via (at 119.75 81.5) (size 0.48) (drill 0.3) (layers "F.Cu" "B.Cu") (free yes) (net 1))
 (via (at 118.25 85.6) (size 0.48) (drill 0.3) (layers "F.Cu" "B.Cu") (free yes) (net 1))
 (via (at 103.6125 79.5) (size 0.48) (drill 0.3) (layers "F.Cu" "B.Cu") (free yes) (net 1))
 (via (at 102.05 82.85) (size 0.48) (drill 0.3) (layers "F.Cu" "B.Cu") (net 1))
 (via (at 103.25 87.1) (size 0.48) (drill 0.3) (layers "F.Cu" "B.Cu") (free yes) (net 1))
 (via (at 108.45 81) (size 0.48) (drill 0.3) (layers "F.Cu" "B.Cu") (free yes) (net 1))
 (via (at 103.65 85.7) (size 0.48) (drill 0.3) (layers "F.Cu" "B.Cu") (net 1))
 (via (at 113.55 82.25) (size 0.48) (drill 0.3) (layers "F.Cu" "B.Cu") (free yes) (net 1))
 (via (at 106 83.8) (size 0.48) (drill 0.3) (layers "F.Cu" "B.Cu") (free yes) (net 1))
 (via (at 120.75 85.55) (size 0.48) (drill 0.3) (layers "F.Cu" "B.Cu") (free yes) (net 1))
 (via (at 118.3 87.1) (size 0.48) (drill 0.3) (layers "F.Cu" "B.Cu") (free yes) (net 1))
 (via (at 125.85 89.3) (size 0.48) (drill 0.3) (layers "F.Cu" "B.Cu") (free yes) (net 1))
 (segment (start 102.275 84.775) (end 104.1875 82.8625) (width 0.3) (layer "F.Cu") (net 3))
 (segment (start 102.06 84.775) (end 102.06 88.04) (width 0.3) (layer "F.Cu") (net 3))
 (segment (start 104.1875 82.8625) (end 104.6 82.8625) (width 0.3) (layer "F.Cu") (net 3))
 (segment (start 114.275 81.4) (end 113.425 80.55) (width 0.3) (layer "F.Cu") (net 2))
 (segment (start 110.55 80.55) (end 109.175 81.925) (width 0.3) (layer "F.Cu") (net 2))
 (segment (start 105.9125 84.775) (end 105.55 85.1375) (width 0.3) (layer "F.Cu") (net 2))
 (segment (start 109.175 81.925) (end 109.175 83.275) (width 0.3) (layer "F.Cu") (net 2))
 (segment (start 110.8 83.275) (end 108.7 83.275) (width 0.3) (layer "F.Cu") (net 2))
 (segment (start 113.425 80.55) (end 110.55 80.55) (width 0.3) (layer "F.Cu") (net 2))
 (segment (start 107.2 84.775) (end 105.9125 84.775) (width 0.3) (layer "F.Cu") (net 2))
 (segment (start 108.7 83.275) (end 107.2 84.775) (width 0.3) (layer "F.Cu") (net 2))
 (segment (start 109.175 83.275) (end 110.8 83.275) (width 0.3) (layer "F.Cu") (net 2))
 (segment (start 114.3 82.95) (end 114.3 81.425) (width 0.3) (layer "F.Cu") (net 2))
 (segment (start 112.4 83.35) (end 110.875 83.35) (width 0.3) (layer "F.Cu") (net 2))
 (segment (start 117 85.725) (end 117 88.24) (width 0.2) (layer "F.Cu") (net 4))
 (segment (start 114.3 84.35) (end 113.5 84.35) (width 0.2) (layer "F.Cu") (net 10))
 (segment (start 113.5 84.35) (end 113.3 84.55) (width 0.2) (layer "F.Cu") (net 10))
 (segment (start 113.3 84.55) (end 113.3 85.25) (width 0.2) (layer "F.Cu") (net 10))
 (via (at 114.3 84.35) (size 0.48) (drill 0.3) (layers "F.Cu" "B.Cu") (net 10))
 (segment (start 114.3 84.35) (end 114.35 84.35) (width 0.2) (layer "B.Cu") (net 10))
 (segment (start 114.35 84.35) (end 114.68 84.68) (width 0.2) (layer "B.Cu") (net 10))
 (segment (start 114.68 84.68) (end 118.52 84.68) (width 0.2) (layer "B.Cu") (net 10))
 (segment (start 118.52 84.68) (end 122.13 88.29) (width 0.2) (layer "B.Cu") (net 10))
 (segment (start 109.43 88.29) (end 111.27 86.45) (width 0.2) (layer "F.Cu") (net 12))
 (segment (start 113.705 86.45) (end 114.3 85.855) (width 0.2) (layer "F.Cu") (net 12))
 (segment (start 114.3 85.855) (end 114.3 85.25) (width 0.2) (layer "F.Cu") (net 12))
 (segment (start 111.27 86.45) (end 113.705 86.45) (width 0.2) (layer "F.Cu") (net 12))
 (segment (start 109.13 86.05) (end 113.55 86.05) (width 0.2) (layer "F.Cu") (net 11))
 (segment (start 106.89 88.29) (end 109.13 86.05) (width 0.2) (layer "F.Cu") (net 11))
 (segment (start 113.55 86.05) (end 113.8 85.8) (width 0.2) (layer "F.Cu") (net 11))
 (segment (start 113.8 85.8) (end 113.8 85.25) (width 0.2) (layer "F.Cu") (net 11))
 (segment (start 116.225 84.85) (end 117 84.075) (width 0.2) (layer "F.Cu") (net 5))
 (segment (start 115.2 84.85) (end 116.225 84.85) (width 0.2) (layer "F.Cu") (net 5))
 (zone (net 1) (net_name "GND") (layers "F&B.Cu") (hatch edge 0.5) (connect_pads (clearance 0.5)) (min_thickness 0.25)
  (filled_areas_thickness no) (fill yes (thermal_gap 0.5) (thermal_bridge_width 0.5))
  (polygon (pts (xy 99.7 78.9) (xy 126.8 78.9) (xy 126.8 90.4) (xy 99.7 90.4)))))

